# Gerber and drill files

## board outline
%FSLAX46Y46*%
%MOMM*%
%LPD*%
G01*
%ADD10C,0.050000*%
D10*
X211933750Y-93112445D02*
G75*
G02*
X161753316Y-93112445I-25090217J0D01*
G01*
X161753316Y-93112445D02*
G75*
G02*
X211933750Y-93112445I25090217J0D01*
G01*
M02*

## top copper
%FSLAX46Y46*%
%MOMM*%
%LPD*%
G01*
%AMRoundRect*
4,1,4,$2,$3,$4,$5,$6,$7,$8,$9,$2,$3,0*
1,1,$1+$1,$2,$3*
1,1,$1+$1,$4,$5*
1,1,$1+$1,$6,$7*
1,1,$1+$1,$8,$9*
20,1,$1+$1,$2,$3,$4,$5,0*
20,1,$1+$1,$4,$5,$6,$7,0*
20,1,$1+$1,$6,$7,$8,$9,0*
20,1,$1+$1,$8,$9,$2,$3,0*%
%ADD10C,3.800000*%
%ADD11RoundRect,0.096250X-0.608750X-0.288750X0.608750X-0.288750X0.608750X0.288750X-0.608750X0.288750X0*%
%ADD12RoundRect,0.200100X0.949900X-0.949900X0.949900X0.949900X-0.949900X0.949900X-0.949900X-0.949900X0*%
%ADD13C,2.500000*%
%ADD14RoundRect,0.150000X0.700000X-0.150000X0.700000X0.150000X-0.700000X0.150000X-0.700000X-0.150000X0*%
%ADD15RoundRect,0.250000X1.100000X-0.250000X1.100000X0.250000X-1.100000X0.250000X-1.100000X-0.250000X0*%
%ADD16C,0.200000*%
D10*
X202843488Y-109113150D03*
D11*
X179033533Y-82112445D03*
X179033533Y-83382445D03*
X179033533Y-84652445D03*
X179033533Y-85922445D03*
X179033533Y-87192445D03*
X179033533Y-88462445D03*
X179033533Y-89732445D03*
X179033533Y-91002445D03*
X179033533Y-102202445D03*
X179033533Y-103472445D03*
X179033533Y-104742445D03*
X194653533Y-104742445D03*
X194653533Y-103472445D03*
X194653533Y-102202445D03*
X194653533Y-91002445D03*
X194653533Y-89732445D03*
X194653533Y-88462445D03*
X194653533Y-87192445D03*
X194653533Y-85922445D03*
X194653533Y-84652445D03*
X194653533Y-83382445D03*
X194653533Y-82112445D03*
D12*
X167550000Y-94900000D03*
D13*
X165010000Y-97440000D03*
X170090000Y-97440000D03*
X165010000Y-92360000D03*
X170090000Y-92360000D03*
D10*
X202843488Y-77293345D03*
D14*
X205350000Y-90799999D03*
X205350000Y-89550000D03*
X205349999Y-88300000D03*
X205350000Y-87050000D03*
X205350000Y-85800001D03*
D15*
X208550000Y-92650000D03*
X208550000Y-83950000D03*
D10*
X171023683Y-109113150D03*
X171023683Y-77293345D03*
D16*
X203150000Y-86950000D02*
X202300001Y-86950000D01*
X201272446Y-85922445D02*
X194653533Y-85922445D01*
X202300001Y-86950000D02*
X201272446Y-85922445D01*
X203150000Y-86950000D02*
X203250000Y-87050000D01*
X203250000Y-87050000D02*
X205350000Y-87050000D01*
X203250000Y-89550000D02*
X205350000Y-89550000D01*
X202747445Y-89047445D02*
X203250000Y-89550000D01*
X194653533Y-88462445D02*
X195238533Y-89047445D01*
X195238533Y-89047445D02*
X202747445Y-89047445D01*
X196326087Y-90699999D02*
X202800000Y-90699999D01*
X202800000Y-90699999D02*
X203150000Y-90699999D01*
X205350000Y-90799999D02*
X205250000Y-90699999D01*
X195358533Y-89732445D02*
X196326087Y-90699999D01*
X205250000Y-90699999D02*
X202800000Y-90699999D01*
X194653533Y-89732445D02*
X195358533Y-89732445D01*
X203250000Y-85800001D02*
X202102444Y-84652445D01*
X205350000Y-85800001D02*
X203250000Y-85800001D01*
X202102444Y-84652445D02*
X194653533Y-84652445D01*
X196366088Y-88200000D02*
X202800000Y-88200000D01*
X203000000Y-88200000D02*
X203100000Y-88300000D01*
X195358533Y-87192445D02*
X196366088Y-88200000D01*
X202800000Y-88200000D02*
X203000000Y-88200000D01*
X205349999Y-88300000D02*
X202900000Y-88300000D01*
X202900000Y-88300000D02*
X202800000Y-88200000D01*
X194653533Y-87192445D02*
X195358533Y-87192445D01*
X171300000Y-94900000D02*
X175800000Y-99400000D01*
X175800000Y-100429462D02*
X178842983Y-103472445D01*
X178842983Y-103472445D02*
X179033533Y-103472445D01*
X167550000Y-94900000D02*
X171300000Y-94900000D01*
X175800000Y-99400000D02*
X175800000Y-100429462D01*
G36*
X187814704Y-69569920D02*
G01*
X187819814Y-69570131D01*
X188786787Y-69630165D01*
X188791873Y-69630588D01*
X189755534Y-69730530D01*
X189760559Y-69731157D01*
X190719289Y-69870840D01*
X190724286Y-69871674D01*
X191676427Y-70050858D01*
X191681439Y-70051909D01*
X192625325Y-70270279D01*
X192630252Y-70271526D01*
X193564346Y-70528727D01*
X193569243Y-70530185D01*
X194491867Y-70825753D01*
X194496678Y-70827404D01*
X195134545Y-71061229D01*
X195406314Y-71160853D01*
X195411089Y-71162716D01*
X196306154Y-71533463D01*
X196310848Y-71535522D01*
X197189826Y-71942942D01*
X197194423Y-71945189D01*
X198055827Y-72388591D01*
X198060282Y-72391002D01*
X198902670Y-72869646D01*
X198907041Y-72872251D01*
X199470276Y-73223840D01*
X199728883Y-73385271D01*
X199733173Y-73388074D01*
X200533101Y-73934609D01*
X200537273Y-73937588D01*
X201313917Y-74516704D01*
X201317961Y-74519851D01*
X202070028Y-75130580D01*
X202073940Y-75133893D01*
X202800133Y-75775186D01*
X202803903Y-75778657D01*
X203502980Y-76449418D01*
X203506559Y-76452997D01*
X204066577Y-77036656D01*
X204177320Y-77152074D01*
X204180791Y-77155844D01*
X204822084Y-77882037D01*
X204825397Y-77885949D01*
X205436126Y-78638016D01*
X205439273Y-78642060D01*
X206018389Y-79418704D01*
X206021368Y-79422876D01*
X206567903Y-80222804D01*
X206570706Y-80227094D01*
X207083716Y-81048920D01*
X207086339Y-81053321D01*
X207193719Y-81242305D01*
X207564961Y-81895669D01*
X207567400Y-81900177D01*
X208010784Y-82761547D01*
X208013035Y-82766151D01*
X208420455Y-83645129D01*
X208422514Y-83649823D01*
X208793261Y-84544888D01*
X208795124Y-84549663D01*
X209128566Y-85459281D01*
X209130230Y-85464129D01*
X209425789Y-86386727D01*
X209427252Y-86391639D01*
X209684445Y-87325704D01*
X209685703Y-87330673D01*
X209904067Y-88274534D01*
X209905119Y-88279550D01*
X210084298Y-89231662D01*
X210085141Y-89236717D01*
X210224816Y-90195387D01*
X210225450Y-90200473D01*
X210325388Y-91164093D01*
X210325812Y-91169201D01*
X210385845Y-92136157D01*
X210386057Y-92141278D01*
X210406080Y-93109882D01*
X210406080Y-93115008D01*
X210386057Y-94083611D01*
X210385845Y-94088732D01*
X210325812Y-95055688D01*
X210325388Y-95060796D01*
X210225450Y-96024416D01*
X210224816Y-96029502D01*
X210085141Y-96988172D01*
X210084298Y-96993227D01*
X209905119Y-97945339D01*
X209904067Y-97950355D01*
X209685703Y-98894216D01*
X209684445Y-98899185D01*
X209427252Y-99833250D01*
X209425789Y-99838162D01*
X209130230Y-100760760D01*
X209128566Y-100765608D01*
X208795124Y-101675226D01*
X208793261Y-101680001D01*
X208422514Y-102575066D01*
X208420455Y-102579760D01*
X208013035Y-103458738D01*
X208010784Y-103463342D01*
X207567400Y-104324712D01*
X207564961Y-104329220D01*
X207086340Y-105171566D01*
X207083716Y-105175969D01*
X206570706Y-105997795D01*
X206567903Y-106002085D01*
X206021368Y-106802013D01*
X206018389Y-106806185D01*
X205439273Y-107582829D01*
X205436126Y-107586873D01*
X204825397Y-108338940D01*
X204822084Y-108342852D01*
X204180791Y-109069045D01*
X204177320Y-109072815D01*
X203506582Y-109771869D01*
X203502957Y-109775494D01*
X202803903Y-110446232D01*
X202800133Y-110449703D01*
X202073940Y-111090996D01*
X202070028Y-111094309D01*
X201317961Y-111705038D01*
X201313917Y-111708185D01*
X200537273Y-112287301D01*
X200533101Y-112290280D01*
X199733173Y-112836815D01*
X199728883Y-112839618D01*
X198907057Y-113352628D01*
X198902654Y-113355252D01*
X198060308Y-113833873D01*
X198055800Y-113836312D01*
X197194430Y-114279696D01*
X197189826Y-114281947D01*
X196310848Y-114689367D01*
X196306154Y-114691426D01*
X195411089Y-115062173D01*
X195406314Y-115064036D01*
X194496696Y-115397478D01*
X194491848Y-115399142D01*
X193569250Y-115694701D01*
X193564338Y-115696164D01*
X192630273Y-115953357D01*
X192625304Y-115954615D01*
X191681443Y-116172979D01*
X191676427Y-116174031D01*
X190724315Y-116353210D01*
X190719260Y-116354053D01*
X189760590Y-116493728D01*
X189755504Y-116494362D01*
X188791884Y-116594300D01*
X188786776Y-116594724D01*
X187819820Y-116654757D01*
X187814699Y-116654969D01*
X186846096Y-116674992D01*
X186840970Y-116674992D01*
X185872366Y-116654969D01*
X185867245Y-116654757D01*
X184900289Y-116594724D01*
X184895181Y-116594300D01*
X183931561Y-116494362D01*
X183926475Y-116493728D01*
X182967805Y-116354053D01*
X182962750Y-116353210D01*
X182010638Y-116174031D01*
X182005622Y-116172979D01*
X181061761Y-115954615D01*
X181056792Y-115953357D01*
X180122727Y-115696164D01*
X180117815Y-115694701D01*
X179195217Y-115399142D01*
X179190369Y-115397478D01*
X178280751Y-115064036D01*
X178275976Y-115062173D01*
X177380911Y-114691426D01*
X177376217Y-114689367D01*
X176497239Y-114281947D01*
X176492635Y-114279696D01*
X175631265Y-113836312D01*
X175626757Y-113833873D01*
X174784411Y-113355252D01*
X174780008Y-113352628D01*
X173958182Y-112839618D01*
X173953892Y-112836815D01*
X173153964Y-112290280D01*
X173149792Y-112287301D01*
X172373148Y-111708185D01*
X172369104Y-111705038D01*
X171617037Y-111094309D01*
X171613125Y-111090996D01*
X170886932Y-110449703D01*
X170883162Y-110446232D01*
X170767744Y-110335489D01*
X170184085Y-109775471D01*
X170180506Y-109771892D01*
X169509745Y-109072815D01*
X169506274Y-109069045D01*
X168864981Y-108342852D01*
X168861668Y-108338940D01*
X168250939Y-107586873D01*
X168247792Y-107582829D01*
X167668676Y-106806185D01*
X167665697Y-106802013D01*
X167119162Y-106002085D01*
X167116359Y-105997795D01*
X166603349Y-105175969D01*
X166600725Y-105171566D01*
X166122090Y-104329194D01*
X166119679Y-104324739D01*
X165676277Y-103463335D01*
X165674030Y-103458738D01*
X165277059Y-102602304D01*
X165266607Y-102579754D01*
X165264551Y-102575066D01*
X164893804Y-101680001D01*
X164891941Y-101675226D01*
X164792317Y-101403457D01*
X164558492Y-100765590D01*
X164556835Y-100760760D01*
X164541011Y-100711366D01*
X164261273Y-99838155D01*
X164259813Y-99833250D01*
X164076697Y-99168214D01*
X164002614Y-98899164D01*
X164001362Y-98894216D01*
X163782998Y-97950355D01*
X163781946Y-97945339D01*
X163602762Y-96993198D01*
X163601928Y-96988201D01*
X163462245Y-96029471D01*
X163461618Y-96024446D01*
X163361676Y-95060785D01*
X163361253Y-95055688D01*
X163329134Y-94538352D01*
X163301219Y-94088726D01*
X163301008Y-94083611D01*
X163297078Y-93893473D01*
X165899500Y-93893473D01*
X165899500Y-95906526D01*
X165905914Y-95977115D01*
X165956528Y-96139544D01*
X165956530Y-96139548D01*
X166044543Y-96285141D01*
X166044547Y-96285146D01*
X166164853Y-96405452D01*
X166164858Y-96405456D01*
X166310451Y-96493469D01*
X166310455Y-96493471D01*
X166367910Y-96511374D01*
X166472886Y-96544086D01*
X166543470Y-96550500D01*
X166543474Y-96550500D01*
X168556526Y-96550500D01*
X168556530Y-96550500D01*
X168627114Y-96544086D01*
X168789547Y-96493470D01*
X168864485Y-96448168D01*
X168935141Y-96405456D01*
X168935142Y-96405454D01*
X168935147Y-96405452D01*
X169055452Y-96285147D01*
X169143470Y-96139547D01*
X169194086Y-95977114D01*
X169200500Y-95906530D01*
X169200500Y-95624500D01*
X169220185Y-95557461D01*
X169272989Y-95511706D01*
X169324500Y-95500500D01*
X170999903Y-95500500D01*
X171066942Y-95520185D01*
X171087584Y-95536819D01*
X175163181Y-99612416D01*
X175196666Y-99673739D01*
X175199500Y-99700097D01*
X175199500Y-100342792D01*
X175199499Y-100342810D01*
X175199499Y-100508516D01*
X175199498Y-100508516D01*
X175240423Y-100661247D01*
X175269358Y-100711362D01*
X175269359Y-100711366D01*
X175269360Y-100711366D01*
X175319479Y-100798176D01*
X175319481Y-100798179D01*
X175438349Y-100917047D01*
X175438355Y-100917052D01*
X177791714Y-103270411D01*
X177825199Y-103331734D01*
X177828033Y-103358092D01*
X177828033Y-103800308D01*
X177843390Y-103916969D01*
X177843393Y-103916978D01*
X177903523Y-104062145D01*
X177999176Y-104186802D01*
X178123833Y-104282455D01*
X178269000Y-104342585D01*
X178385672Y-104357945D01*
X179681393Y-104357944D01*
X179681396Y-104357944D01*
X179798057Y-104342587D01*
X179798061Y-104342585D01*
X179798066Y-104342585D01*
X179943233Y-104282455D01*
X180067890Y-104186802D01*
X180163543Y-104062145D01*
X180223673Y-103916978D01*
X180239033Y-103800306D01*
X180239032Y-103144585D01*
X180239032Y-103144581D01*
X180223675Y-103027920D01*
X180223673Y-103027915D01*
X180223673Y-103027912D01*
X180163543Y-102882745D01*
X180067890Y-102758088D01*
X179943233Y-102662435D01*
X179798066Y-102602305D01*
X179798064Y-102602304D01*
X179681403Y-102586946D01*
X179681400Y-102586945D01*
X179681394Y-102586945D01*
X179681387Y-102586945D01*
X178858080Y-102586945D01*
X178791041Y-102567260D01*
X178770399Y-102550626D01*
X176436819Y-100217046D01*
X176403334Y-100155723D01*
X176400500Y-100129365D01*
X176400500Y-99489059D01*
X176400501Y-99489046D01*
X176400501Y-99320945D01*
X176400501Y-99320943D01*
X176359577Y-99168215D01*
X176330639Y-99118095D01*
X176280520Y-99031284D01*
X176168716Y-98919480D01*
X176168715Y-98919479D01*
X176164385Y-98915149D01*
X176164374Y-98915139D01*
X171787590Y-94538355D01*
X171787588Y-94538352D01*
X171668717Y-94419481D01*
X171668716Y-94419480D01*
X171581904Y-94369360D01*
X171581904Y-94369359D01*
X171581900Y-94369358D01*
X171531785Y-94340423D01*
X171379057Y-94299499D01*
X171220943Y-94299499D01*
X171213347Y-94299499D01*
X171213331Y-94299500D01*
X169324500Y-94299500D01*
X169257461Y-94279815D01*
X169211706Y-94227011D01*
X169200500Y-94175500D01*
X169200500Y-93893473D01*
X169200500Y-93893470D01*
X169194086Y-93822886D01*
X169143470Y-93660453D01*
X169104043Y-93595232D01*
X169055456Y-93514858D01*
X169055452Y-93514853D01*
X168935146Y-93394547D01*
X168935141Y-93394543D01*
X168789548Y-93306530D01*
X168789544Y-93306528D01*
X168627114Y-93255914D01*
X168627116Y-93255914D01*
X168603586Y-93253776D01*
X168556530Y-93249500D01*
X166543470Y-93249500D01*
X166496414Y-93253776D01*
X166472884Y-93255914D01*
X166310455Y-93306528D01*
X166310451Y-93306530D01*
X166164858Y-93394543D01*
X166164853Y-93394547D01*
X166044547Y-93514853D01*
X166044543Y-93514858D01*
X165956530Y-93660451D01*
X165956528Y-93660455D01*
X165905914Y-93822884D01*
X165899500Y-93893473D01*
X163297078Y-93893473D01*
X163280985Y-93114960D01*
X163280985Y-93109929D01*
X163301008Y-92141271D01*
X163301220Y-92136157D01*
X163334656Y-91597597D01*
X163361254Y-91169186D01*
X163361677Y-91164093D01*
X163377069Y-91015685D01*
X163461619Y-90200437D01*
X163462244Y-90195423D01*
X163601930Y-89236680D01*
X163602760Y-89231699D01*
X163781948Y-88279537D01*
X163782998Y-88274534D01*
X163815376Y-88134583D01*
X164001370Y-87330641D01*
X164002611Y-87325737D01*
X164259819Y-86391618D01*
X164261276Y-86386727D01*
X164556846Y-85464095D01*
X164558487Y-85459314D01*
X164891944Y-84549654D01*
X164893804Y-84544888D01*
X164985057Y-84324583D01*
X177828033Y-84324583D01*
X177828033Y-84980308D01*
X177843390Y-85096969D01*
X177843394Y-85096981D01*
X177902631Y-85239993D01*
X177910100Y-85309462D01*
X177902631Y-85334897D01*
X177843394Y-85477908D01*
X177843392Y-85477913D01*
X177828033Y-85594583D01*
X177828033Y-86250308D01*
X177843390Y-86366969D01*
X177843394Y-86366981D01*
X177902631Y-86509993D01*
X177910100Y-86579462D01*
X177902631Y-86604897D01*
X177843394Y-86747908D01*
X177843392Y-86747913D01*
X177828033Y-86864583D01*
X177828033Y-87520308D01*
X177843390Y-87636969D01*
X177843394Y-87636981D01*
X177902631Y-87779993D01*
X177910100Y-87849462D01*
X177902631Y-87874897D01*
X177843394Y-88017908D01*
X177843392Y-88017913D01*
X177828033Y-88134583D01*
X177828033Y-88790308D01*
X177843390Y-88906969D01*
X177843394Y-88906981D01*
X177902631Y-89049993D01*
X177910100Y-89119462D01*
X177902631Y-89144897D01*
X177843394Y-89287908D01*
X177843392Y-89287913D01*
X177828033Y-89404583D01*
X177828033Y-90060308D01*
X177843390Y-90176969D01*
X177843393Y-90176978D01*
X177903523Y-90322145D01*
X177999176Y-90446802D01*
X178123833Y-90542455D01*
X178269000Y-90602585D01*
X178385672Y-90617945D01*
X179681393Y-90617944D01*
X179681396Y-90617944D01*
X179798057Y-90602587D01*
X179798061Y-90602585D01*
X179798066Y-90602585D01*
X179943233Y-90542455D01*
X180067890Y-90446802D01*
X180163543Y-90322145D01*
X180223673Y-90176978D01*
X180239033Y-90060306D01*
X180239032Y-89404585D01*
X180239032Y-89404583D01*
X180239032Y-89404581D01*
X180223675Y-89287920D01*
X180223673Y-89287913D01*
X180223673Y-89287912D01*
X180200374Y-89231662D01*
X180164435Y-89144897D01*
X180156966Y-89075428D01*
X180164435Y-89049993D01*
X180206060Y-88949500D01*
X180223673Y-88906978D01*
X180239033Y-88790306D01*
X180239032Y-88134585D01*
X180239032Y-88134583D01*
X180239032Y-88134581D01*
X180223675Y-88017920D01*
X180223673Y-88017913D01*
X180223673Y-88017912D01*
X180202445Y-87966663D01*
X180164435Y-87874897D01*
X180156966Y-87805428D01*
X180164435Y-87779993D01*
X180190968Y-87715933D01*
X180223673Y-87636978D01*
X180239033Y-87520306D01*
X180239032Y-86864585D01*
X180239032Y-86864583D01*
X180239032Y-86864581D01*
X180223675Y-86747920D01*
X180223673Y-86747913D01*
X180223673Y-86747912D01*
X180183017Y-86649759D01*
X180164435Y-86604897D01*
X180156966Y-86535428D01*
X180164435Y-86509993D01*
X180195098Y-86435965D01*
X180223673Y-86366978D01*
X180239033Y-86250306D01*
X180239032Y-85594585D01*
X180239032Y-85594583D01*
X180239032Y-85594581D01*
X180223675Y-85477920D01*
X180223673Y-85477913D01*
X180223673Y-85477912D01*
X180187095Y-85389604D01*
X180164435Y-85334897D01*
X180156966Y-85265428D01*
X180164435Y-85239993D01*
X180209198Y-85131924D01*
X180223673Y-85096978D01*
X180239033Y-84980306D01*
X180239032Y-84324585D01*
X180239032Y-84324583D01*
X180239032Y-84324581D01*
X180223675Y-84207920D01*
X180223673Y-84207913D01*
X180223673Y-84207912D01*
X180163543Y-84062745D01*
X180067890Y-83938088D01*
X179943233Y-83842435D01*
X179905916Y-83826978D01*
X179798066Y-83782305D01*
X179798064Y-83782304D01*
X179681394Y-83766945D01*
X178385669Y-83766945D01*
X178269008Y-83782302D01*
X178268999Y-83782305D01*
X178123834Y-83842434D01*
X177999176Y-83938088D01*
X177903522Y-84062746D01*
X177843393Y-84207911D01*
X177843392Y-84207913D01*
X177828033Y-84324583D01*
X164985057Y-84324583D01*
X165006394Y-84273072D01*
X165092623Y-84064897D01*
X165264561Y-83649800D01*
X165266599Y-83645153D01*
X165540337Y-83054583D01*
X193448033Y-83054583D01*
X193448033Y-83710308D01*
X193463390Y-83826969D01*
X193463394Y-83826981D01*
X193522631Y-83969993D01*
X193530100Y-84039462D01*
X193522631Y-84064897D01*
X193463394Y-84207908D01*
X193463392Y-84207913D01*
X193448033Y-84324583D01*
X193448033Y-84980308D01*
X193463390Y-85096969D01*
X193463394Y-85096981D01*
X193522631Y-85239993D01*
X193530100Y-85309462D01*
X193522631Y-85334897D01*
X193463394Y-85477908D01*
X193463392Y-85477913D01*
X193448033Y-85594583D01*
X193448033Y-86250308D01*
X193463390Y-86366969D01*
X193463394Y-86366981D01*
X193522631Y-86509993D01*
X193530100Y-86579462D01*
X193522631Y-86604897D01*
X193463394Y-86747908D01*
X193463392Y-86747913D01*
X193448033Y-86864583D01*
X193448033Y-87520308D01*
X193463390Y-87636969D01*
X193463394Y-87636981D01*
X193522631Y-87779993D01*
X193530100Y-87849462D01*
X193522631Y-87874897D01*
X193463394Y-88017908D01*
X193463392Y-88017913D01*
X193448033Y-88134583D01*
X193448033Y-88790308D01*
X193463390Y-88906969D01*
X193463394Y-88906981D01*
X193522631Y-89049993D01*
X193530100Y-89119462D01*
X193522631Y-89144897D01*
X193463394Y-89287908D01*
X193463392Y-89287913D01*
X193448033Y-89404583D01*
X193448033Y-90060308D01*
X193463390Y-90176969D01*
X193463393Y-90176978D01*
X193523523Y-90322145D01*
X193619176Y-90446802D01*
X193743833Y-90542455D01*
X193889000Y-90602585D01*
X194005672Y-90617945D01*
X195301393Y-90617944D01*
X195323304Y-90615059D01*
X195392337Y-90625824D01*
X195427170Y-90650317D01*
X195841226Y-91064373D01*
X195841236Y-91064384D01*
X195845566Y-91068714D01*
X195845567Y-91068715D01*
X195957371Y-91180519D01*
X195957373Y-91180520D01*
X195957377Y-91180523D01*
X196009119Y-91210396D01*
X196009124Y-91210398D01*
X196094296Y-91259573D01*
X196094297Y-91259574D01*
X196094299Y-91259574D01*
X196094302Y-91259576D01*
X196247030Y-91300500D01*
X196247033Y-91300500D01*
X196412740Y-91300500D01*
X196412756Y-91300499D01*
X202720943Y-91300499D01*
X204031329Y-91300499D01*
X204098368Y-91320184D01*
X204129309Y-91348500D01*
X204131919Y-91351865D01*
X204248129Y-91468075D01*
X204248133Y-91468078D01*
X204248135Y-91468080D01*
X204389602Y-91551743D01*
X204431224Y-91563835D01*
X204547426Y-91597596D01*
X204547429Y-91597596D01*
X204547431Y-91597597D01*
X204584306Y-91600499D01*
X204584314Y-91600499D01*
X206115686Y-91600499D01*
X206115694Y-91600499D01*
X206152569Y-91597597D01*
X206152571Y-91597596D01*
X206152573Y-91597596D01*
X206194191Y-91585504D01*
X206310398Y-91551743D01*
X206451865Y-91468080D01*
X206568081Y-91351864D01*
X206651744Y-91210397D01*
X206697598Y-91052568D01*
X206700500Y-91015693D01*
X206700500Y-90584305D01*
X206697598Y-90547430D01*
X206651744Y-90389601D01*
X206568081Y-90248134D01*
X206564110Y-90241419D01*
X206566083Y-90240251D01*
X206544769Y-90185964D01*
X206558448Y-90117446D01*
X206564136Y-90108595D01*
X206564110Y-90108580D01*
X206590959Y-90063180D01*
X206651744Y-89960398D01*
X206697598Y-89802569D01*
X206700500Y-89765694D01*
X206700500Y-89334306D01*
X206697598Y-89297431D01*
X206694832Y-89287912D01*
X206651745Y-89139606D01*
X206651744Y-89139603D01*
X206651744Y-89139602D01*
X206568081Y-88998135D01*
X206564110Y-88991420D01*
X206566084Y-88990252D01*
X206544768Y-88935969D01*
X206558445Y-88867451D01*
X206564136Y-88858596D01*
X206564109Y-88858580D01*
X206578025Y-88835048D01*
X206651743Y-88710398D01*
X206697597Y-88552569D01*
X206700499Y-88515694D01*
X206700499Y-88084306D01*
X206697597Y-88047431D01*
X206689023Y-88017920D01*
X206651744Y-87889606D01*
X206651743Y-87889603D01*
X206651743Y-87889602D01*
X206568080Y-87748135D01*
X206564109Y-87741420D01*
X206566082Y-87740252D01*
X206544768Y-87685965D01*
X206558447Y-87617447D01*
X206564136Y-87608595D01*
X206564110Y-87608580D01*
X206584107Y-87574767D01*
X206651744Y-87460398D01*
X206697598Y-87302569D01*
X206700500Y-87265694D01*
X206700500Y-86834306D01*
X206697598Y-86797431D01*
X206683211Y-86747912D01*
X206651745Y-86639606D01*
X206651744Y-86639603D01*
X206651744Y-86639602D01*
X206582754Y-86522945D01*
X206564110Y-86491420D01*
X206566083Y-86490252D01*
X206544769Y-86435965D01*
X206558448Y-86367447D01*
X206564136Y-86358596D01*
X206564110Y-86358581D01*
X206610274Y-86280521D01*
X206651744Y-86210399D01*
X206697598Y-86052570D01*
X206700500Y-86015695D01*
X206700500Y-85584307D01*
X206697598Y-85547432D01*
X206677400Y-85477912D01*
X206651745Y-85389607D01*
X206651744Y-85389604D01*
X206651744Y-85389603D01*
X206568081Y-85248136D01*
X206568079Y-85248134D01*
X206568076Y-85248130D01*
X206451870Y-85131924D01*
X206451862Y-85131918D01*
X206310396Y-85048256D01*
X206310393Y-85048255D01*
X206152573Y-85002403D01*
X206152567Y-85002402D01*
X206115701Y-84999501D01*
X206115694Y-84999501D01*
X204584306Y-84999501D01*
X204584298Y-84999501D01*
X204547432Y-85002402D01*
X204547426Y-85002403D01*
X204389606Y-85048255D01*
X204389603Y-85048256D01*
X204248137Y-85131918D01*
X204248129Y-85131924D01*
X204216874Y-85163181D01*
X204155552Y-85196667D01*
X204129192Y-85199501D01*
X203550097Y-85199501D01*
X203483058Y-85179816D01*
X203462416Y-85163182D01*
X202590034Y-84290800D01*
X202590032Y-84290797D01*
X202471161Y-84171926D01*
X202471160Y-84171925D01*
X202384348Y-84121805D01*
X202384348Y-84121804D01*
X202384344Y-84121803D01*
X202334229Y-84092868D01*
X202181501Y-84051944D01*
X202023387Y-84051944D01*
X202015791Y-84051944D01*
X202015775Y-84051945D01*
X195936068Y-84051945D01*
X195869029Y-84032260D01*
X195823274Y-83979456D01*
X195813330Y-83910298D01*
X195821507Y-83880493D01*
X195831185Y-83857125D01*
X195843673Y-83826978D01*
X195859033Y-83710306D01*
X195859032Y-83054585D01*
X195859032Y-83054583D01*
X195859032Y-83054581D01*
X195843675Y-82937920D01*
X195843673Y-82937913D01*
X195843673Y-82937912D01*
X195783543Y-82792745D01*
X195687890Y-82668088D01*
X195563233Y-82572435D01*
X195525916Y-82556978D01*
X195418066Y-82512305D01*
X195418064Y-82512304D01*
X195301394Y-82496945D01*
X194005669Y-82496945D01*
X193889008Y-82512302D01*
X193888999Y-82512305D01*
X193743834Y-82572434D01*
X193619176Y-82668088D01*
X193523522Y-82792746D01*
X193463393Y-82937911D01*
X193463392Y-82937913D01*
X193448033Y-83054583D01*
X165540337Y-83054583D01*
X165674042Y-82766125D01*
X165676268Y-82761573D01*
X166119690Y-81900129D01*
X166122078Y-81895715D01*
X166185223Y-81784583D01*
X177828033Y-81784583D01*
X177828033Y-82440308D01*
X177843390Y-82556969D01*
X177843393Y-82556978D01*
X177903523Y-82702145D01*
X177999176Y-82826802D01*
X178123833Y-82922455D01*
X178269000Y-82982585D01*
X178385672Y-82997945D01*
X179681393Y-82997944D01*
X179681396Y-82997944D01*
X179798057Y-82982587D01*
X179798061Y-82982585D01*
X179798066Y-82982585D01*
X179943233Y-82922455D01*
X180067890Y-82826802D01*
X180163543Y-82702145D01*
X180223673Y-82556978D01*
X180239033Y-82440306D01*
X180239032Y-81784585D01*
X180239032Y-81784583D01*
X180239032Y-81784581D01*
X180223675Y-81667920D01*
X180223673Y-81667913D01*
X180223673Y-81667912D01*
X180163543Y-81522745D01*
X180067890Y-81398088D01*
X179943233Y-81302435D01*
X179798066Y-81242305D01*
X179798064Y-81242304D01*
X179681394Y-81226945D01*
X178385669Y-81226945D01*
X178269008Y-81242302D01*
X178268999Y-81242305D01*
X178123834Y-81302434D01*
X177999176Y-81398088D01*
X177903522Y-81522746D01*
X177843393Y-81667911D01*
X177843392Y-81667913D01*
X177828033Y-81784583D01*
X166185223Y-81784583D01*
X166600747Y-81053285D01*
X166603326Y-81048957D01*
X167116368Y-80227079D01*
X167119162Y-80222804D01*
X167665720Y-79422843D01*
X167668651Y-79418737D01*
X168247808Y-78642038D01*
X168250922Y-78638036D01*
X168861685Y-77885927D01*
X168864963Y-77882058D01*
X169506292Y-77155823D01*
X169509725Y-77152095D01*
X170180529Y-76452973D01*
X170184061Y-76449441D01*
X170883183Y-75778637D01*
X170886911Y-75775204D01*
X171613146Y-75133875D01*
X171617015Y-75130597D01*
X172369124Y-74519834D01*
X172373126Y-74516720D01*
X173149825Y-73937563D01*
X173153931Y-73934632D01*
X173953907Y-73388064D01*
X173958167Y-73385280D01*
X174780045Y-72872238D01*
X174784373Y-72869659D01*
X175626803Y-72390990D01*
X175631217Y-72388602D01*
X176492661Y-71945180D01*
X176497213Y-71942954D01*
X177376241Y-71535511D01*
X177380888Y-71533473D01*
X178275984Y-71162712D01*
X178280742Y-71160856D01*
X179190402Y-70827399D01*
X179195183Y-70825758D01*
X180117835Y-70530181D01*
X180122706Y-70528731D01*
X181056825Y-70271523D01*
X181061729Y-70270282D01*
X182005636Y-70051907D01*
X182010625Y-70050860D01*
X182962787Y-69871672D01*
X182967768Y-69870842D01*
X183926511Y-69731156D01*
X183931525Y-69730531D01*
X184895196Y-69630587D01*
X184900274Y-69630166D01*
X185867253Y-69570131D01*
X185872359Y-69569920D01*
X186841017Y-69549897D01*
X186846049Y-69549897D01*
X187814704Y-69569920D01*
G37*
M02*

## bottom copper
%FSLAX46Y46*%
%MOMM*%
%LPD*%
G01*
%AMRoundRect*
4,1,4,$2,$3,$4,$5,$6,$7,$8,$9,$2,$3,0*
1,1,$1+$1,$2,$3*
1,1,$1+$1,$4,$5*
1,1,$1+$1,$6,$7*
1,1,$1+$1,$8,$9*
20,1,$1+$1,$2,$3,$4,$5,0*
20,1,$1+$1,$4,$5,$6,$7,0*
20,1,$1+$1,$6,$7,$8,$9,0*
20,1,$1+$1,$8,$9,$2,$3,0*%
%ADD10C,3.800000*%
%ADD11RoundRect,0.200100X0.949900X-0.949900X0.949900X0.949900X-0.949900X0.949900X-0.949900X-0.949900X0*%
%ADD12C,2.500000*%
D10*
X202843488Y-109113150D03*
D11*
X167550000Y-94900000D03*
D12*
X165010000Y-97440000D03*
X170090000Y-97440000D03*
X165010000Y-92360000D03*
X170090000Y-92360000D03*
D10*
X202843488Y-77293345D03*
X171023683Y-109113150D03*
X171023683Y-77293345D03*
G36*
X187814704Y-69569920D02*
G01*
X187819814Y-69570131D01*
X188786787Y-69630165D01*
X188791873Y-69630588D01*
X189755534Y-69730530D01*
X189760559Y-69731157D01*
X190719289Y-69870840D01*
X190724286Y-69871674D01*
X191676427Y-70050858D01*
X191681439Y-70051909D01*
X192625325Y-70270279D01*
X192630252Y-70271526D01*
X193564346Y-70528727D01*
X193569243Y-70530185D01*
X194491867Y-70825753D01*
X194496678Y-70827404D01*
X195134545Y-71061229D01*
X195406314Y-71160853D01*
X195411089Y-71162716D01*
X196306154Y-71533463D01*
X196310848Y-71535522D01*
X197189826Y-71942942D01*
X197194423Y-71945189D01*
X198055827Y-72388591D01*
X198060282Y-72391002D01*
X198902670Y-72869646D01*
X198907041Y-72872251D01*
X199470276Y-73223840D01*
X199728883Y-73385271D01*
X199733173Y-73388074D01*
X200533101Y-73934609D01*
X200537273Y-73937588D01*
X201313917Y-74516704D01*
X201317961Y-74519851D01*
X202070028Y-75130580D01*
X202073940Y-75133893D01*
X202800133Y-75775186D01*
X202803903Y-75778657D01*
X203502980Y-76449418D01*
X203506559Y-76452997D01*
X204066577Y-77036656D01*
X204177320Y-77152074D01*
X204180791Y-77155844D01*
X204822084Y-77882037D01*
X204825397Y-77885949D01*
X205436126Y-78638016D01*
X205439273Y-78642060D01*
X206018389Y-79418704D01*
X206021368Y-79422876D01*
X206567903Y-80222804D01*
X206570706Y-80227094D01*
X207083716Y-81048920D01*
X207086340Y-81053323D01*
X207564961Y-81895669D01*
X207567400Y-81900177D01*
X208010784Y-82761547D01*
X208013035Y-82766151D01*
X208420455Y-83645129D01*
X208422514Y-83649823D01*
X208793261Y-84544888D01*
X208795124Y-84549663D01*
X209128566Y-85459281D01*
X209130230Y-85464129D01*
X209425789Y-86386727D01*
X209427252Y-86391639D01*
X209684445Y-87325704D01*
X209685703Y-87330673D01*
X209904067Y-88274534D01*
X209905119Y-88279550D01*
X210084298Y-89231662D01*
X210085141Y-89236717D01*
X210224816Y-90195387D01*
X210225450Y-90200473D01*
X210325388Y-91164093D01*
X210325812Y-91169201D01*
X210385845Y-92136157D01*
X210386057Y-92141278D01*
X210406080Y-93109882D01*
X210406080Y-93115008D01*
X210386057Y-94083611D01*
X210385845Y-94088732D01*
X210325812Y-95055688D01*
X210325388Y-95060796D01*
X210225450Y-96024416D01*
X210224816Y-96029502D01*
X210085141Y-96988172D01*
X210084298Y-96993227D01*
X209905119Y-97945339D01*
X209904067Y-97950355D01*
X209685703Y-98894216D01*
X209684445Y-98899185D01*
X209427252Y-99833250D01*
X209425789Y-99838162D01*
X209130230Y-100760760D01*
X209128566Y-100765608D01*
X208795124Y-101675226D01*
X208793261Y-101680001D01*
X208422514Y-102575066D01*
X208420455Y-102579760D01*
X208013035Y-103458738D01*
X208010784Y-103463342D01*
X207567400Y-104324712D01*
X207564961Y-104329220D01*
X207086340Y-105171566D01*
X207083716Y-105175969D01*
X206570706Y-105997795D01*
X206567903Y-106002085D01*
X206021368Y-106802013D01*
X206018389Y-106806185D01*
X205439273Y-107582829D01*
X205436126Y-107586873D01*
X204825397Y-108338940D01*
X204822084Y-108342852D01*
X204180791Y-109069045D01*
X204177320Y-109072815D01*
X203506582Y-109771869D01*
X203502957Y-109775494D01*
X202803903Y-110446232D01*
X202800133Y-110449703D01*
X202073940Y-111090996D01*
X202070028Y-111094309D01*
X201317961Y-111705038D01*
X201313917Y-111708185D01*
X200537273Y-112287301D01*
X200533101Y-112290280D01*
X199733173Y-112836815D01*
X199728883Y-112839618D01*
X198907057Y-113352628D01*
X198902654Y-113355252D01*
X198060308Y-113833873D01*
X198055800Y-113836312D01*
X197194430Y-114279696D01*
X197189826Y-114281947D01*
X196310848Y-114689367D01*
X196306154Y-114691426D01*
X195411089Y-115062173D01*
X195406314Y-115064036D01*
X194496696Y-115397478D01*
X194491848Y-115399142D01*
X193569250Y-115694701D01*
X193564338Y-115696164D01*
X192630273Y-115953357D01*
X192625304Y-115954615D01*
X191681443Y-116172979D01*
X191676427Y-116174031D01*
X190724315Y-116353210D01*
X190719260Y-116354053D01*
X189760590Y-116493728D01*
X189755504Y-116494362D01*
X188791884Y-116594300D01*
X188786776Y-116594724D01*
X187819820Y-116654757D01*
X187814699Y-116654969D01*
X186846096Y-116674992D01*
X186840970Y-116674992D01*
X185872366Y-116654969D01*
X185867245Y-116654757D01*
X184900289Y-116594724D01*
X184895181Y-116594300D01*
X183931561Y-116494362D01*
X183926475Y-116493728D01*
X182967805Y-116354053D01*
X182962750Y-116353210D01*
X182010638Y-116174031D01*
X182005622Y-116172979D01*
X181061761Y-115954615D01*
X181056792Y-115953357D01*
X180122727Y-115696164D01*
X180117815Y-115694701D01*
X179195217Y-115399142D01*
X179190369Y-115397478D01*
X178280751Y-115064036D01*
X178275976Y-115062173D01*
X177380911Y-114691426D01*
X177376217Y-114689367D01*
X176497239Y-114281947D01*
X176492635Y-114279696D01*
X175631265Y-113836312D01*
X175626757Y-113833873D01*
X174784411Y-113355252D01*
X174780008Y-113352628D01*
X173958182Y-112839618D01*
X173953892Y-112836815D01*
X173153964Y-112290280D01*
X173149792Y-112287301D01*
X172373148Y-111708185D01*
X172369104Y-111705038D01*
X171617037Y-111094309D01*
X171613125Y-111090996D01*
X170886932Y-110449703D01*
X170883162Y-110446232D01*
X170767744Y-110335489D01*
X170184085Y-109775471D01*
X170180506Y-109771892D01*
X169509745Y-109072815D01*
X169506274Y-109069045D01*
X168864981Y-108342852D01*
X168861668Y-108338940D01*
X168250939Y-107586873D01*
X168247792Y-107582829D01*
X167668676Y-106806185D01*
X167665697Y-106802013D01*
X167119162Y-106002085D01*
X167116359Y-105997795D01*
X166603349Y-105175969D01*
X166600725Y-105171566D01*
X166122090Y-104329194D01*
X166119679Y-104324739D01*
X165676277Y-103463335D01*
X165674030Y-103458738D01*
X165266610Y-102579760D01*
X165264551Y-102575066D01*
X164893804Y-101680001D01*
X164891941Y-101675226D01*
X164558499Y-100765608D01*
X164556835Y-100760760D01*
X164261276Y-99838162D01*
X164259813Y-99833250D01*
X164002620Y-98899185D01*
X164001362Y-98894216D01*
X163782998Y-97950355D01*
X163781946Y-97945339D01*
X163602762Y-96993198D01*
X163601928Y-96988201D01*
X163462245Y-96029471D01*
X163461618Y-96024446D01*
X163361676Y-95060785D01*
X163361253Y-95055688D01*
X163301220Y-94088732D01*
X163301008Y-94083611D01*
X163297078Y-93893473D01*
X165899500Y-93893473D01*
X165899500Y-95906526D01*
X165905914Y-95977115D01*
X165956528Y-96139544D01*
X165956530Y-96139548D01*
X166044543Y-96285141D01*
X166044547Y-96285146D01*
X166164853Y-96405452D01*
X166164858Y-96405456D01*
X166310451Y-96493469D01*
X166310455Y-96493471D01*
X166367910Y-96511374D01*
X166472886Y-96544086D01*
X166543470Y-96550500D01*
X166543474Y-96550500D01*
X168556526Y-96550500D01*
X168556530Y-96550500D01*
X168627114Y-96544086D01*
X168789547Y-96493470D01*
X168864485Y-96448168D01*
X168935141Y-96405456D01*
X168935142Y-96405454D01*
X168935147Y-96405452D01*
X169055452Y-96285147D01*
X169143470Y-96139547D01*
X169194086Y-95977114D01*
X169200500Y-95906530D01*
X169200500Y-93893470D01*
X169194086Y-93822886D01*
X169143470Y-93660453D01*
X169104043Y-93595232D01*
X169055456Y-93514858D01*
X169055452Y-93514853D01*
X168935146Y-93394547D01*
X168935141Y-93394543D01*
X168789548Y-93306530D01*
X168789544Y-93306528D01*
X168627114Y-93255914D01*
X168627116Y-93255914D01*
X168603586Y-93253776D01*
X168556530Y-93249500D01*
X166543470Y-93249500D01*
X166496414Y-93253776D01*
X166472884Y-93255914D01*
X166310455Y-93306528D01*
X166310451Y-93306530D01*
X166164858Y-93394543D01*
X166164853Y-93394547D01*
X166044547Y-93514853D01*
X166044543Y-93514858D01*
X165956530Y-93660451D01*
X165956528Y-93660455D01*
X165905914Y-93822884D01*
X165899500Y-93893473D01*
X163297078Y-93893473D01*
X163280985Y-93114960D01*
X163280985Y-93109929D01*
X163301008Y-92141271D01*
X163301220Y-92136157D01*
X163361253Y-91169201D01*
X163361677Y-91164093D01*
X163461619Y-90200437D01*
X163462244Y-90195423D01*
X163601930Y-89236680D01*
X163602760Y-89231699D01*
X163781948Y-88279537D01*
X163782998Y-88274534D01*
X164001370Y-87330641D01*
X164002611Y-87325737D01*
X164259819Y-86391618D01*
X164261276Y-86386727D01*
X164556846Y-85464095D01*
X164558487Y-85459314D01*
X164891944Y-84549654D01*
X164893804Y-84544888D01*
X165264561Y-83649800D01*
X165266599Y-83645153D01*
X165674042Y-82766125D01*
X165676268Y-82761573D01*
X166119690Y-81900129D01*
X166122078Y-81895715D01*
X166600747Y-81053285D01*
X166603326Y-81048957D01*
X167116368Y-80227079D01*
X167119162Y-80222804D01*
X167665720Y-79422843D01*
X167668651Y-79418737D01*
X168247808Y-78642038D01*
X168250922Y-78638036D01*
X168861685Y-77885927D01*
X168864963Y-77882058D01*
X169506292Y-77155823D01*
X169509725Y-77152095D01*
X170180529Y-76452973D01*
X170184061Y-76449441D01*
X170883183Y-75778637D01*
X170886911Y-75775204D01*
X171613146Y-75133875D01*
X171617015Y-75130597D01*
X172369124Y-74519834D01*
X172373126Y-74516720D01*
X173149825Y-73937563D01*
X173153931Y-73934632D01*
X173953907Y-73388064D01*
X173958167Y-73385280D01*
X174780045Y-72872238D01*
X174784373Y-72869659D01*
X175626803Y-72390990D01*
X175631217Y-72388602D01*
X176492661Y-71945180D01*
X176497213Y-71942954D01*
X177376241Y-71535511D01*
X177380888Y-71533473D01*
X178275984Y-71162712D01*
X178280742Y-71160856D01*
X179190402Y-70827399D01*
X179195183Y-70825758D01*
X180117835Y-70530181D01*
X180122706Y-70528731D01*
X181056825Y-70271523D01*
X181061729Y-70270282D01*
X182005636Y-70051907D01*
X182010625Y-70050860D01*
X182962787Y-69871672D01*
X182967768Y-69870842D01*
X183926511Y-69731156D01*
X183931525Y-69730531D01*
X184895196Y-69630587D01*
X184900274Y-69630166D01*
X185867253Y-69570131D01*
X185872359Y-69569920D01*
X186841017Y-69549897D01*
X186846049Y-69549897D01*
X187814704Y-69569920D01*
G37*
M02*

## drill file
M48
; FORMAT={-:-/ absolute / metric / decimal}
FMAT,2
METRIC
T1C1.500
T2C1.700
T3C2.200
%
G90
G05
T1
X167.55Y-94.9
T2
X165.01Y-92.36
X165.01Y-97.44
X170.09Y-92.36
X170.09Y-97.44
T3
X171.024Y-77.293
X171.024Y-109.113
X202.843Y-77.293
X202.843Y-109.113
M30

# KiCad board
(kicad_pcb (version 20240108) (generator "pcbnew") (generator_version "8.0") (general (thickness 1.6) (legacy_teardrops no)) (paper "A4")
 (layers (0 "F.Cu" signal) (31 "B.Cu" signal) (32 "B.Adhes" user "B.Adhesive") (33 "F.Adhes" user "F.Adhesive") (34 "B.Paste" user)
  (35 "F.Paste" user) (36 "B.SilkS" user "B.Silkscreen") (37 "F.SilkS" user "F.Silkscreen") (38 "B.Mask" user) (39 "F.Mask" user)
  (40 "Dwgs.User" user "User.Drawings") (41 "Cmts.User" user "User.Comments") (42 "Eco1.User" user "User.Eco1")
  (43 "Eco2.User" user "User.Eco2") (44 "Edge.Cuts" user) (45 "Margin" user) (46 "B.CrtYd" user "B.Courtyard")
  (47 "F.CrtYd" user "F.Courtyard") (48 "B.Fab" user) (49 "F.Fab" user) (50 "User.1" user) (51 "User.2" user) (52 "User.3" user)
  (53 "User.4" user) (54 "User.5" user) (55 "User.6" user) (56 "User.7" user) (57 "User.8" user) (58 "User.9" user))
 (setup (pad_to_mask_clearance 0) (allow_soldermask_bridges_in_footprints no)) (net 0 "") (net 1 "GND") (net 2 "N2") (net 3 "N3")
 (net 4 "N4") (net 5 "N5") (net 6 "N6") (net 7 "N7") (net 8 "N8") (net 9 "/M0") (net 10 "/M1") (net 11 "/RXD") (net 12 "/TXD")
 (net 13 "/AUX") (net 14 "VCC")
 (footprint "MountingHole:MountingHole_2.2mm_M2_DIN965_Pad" (layer "F.Cu") (at 202.843488 109.11315)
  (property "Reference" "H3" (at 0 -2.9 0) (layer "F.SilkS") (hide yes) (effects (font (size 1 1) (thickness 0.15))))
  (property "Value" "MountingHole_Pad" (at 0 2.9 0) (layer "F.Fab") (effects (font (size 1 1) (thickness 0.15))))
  (pad "1" thru_hole circle (at 0 0) (size 3.8 3.8) (drill 2.2) (layers "*.Cu" "*.Mask") (remove_unused_layers no) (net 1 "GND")))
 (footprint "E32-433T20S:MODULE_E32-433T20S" (layer "F.Cu") (at 186.843533 93.112445)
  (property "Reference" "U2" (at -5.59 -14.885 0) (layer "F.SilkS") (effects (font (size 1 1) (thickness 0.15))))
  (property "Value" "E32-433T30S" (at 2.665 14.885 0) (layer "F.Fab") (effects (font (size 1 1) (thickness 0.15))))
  (pad "1" smd roundrect (at -7.81 -11) (size 1.41 0.77) (layers "F.Cu" "F.Paste" "F.Mask") (roundrect_rratio 0.125) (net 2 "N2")
   (solder_mask_margin 0.102))
  (pad "2" smd roundrect (at -7.81 -9.73) (size 1.41 0.77) (layers "F.Cu" "F.Paste" "F.Mask") (roundrect_rratio 0.125) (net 1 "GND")
   (solder_mask_margin 0.102))
  (pad "3" smd roundrect (at -7.81 -8.46) (size 1.41 0.77) (layers "F.Cu" "F.Paste" "F.Mask") (roundrect_rratio 0.125) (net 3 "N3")
   (solder_mask_margin 0.102))
  (pad "4" smd roundrect (at -7.81 -7.19) (size 1.41 0.77) (layers "F.Cu" "F.Paste" "F.Mask") (roundrect_rratio 0.125) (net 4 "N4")
   (solder_mask_margin 0.102))
  (pad "5" smd roundrect (at -7.81 -5.92) (size 1.41 0.77) (layers "F.Cu" "F.Paste" "F.Mask") (roundrect_rratio 0.125) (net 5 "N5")
   (solder_mask_margin 0.102))
  (pad "6" smd roundrect (at -7.81 -4.65) (size 1.41 0.77) (layers "F.Cu" "F.Paste" "F.Mask") (roundrect_rratio 0.125) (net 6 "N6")
   (solder_mask_margin 0.102))
  (pad "7" smd roundrect (at -7.81 -3.38) (size 1.41 0.77) (layers "F.Cu" "F.Paste" "F.Mask") (roundrect_rratio 0.125) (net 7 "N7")
   (solder_mask_margin 0.102))
  (pad "8" smd roundrect (at -7.81 -2.11) (size 1.41 0.77) (layers "F.Cu" "F.Paste" "F.Mask") (roundrect_rratio 0.125) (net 1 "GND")
   (solder_mask_margin 0.102))
  (pad "11" smd roundrect (at -7.81 9.09) (size 1.41 0.77) (layers "F.Cu" "F.Paste" "F.Mask") (roundrect_rratio 0.125) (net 1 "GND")
   (solder_mask_margin 0.102))
  (pad "12" smd roundrect (at -7.81 10.36) (size 1.41 0.77) (layers "F.Cu" "F.Paste" "F.Mask") (roundrect_rratio 0.125) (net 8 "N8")
   (solder_mask_margin 0.102))
  (pad "13" smd roundrect (at -7.81 11.63) (size 1.41 0.77) (layers "F.Cu" "F.Paste" "F.Mask") (roundrect_rratio 0.125) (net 1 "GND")
   (solder_mask_margin 0.102))
  (pad "14" smd roundrect (at 7.81 11.63) (size 1.41 0.77) (layers "F.Cu" "F.Paste" "F.Mask") (roundrect_rratio 0.125) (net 1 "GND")
   (solder_mask_margin 0.102))
  (pad "15" smd roundrect (at 7.81 10.36) (size 1.41 0.77) (layers "F.Cu" "F.Paste" "F.Mask") (roundrect_rratio 0.125) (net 1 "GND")
   (solder_mask_margin 0.102))
  (pad "16" smd roundrect (at 7.81 9.09) (size 1.41 0.77) (layers "F.Cu" "F.Paste" "F.Mask") (roundrect_rratio 0.125) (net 1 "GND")
   (solder_mask_margin 0.102))
  (pad "19" smd roundrect (at 7.81 -2.11) (size 1.41 0.77) (layers "F.Cu" "F.Paste" "F.Mask") (roundrect_rratio 0.125) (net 1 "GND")
   (solder_mask_margin 0.102))
  (pad "20" smd roundrect (at 7.81 -3.38) (size 1.41 0.77) (layers "F.Cu" "F.Paste" "F.Mask") (roundrect_rratio 0.125) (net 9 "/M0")
   (solder_mask_margin 0.102))
  (pad "21" smd roundrect (at 7.81 -4.65) (size 1.41 0.77) (layers "F.Cu" "F.Paste" "F.Mask") (roundrect_rratio 0.125) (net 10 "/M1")
   (solder_mask_margin 0.102))
  (pad "22" smd roundrect (at 7.81 -5.92) (size 1.41 0.77) (layers "F.Cu" "F.Paste" "F.Mask") (roundrect_rratio 0.125) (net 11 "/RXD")
   (solder_mask_margin 0.102))
  (pad "23" smd roundrect (at 7.81 -7.19) (size 1.41 0.77) (layers "F.Cu" "F.Paste" "F.Mask") (roundrect_rratio 0.125) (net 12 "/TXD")
   (solder_mask_margin 0.102))
  (pad "24" smd roundrect (at 7.81 -8.46) (size 1.41 0.77) (layers "F.Cu" "F.Paste" "F.Mask") (roundrect_rratio 0.125) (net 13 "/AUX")
   (solder_mask_margin 0.102))
  (pad "25" smd roundrect (at 7.81 -9.73) (size 1.41 0.77) (layers "F.Cu" "F.Paste" "F.Mask") (roundrect_rratio 0.125) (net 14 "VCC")
   (solder_mask_margin 0.102))
  (pad "26" smd roundrect (at 7.81 -11) (size 1.41 0.77) (layers "F.Cu" "F.Paste" "F.Mask") (roundrect_rratio 0.125) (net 1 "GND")
   (solder_mask_margin 0.102)))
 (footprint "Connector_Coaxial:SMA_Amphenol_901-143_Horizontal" (layer "F.Cu") (at 167.55 94.9 90)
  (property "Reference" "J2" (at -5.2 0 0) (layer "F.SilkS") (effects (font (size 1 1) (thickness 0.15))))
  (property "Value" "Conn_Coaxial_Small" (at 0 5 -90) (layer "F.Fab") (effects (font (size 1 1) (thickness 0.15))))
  (pad "1" thru_hole roundrect (at 0 0 90) (size 2.3 2.3) (drill 1.5) (layers "*.Cu" "*.Mask") (remove_unused_layers yes)
   (keep_end_layers yes) (zone_layer_connections) (roundrect_rratio 0.087) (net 8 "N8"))
  (pad "2" thru_hole circle (at -2.54 -2.54 90) (size 2.5 2.5) (drill 1.7) (layers "*.Cu" "*.Mask") (remove_unused_layers yes)
   (keep_end_layers yes) (zone_layer_connections) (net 1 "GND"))
  (pad "2" thru_hole circle (at -2.54 2.54 90) (size 2.5 2.5) (drill 1.7) (layers "*.Cu" "*.Mask") (remove_unused_layers yes)
   (keep_end_layers yes) (zone_layer_connections) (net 1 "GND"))
  (pad "2" thru_hole circle (at 2.54 -2.54 90) (size 2.5 2.5) (drill 1.7) (layers "*.Cu" "*.Mask") (remove_unused_layers yes)
   (keep_end_layers yes) (zone_layer_connections) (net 1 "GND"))
  (pad "2" thru_hole circle (at 2.54 2.54 90) (size 2.5 2.5) (drill 1.7) (layers "*.Cu" "*.Mask") (remove_unused_layers yes)
   (keep_end_layers yes) (zone_layer_connections) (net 1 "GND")))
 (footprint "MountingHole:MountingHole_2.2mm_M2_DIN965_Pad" (layer "F.Cu") (at 202.843488 77.293345)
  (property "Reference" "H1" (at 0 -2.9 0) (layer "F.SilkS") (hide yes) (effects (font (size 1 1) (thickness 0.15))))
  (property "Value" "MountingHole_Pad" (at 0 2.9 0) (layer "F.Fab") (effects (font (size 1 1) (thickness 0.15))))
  (pad "1" thru_hole circle (at 0 0) (size 3.8 3.8) (drill 2.2) (layers "*.Cu" "*.Mask") (remove_unused_layers no) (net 1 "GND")))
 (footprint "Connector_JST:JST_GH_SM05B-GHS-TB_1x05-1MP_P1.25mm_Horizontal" (layer "F.Cu") (at 207.2 88.3 90)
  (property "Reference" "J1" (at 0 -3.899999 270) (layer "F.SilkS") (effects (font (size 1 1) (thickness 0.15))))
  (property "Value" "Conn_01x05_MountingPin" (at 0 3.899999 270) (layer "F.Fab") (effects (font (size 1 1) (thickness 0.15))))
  (pad "1" smd roundrect (at -2.499999 -1.85 90) (size 0.6 1.7) (layers "F.Cu" "F.Paste" "F.Mask") (roundrect_rratio 0.25) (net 9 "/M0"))
  (pad "2" smd roundrect (at -1.25 -1.85 90) (size 0.6 1.7) (layers "F.Cu" "F.Paste" "F.Mask") (roundrect_rratio 0.25) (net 10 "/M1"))
  (pad "3" smd roundrect (at 0 -1.850001 90) (size 0.6 1.7) (layers "F.Cu" "F.Paste" "F.Mask") (roundrect_rratio 0.25) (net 11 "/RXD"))
  (pad "4" smd roundrect (at 1.25 -1.85 90) (size 0.6 1.7) (layers "F.Cu" "F.Paste" "F.Mask") (roundrect_rratio 0.25) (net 12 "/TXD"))
  (pad "5" smd roundrect (at 2.499999 -1.85 90) (size 0.6 1.7) (layers "F.Cu" "F.Paste" "F.Mask") (roundrect_rratio 0.25) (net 13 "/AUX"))
  (pad "MP" smd roundrect (at -4.35 1.35 90) (size 1 2.7) (layers "F.Cu" "F.Paste" "F.Mask") (roundrect_rratio 0.25) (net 1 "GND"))
  (pad "MP" smd roundrect (at 4.35 1.35 90) (size 1 2.7) (layers "F.Cu" "F.Paste" "F.Mask") (roundrect_rratio 0.25) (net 1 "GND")))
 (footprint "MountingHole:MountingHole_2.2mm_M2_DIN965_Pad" (layer "F.Cu") (at 171.023683 109.11315)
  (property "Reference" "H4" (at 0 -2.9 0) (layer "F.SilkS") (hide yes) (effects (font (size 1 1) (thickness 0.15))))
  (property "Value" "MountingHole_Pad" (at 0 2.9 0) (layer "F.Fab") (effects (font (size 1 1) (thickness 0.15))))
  (pad "1" thru_hole circle (at 0 0) (size 3.8 3.8) (drill 2.2) (layers "*.Cu" "*.Mask") (remove_unused_layers no) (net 1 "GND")))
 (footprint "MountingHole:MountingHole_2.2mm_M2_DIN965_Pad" (layer "F.Cu") (at 171.023683 77.293345)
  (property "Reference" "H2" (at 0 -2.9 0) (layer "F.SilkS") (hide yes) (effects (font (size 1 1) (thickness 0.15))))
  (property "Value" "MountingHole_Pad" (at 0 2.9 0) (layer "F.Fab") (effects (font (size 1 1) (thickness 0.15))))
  (pad "1" thru_hole circle (at 0 0) (size 3.8 3.8) (drill 2.2) (layers "*.Cu" "*.Mask") (remove_unused_layers no) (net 1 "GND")))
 (gr_circle (center 186.843533 93.112445) (end 211.933586 93.203248) (stroke (width 0.05) (type default)) (fill none) (layer "Edge.Cuts"))
 (segment (start 203.15 86.95) (end 202.300001 86.95) (width 0.2) (layer "F.Cu") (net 12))
 (segment (start 201.272446 85.922445) (end 194.653533 85.922445) (width 0.2) (layer "F.Cu") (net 12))
 (segment (start 202.300001 86.95) (end 201.272446 85.922445) (width 0.2) (layer "F.Cu") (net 12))
 (segment (start 203.15 86.95) (end 203.25 87.05) (width 0.2) (layer "F.Cu") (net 12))
 (segment (start 203.25 87.05) (end 205.35 87.05) (width 0.2) (layer "F.Cu") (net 12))
 (segment (start 203.25 89.55) (end 205.35 89.55) (width 0.2) (layer "F.Cu") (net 10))
 (segment (start 202.747445 89.047445) (end 203.25 89.55) (width 0.2) (layer "F.Cu") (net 10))
 (segment (start 194.653533 88.462445) (end 195.238533 89.047445) (width 0.2) (layer "F.Cu") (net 10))
 (segment (start 195.238533 89.047445) (end 202.747445 89.047445) (width 0.2) (layer "F.Cu") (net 10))
 (segment (start 196.326087 90.699999) (end 202.8 90.699999) (width 0.2) (layer "F.Cu") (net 9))
 (segment (start 202.8 90.699999) (end 203.15 90.699999) (width 0.2) (layer "F.Cu") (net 9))
 (segment (start 205.35 90.799999) (end 205.25 90.699999) (width 0.2) (layer "F.Cu") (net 9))
 (segment (start 195.358533 89.732445) (end 196.326087 90.699999) (width 0.2) (layer "F.Cu") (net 9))
 (segment (start 205.25 90.699999) (end 202.8 90.699999) (width 0.2) (layer "F.Cu") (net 9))
 (segment (start 194.653533 89.732445) (end 195.358533 89.732445) (width 0.2) (layer "F.Cu") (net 9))
 (segment (start 203.25 85.800001) (end 202.102444 84.652445) (width 0.2) (layer "F.Cu") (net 13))
 (segment (start 205.35 85.800001) (end 203.25 85.800001) (width 0.2) (layer "F.Cu") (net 13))
 (segment (start 202.102444 84.652445) (end 194.653533 84.652445) (width 0.2) (layer "F.Cu") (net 13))
 (segment (start 196.366088 88.2) (end 202.8 88.2) (width 0.2) (layer "F.Cu") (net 11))
 (segment (start 203 88.2) (end 203.1 88.3) (width 0.2) (layer "F.Cu") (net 11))
 (segment (start 195.358533 87.192445) (end 196.366088 88.2) (width 0.2) (layer "F.Cu") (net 11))
 (segment (start 202.8 88.2) (end 203 88.2) (width 0.2) (layer "F.Cu") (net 11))
 (segment (start 205.349999 88.3) (end 202.9 88.3) (width 0.2) (layer "F.Cu") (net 11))
 (segment (start 202.9 88.3) (end 202.8 88.2) (width 0.2) (layer "F.Cu") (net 11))
 (segment (start 194.653533 87.192445) (end 195.358533 87.192445) (width 0.2) (layer "F.Cu") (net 11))
 (segment (start 171.3 94.9) (end 175.8 99.4) (width 0.2) (layer "F.Cu") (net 8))
 (segment (start 175.8 100.429462) (end 178.842983 103.472445) (width 0.2) (layer "F.Cu") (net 8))
 (segment (start 178.842983 103.472445) (end 179.033533 103.472445) (width 0.2) (layer "F.Cu") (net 8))
 (segment (start 167.55 94.9) (end 171.3 94.9) (width 0.2) (layer "F.Cu") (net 8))
 (segment (start 175.8 99.4) (end 175.8 100.429462) (width 0.2) (layer "F.Cu") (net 8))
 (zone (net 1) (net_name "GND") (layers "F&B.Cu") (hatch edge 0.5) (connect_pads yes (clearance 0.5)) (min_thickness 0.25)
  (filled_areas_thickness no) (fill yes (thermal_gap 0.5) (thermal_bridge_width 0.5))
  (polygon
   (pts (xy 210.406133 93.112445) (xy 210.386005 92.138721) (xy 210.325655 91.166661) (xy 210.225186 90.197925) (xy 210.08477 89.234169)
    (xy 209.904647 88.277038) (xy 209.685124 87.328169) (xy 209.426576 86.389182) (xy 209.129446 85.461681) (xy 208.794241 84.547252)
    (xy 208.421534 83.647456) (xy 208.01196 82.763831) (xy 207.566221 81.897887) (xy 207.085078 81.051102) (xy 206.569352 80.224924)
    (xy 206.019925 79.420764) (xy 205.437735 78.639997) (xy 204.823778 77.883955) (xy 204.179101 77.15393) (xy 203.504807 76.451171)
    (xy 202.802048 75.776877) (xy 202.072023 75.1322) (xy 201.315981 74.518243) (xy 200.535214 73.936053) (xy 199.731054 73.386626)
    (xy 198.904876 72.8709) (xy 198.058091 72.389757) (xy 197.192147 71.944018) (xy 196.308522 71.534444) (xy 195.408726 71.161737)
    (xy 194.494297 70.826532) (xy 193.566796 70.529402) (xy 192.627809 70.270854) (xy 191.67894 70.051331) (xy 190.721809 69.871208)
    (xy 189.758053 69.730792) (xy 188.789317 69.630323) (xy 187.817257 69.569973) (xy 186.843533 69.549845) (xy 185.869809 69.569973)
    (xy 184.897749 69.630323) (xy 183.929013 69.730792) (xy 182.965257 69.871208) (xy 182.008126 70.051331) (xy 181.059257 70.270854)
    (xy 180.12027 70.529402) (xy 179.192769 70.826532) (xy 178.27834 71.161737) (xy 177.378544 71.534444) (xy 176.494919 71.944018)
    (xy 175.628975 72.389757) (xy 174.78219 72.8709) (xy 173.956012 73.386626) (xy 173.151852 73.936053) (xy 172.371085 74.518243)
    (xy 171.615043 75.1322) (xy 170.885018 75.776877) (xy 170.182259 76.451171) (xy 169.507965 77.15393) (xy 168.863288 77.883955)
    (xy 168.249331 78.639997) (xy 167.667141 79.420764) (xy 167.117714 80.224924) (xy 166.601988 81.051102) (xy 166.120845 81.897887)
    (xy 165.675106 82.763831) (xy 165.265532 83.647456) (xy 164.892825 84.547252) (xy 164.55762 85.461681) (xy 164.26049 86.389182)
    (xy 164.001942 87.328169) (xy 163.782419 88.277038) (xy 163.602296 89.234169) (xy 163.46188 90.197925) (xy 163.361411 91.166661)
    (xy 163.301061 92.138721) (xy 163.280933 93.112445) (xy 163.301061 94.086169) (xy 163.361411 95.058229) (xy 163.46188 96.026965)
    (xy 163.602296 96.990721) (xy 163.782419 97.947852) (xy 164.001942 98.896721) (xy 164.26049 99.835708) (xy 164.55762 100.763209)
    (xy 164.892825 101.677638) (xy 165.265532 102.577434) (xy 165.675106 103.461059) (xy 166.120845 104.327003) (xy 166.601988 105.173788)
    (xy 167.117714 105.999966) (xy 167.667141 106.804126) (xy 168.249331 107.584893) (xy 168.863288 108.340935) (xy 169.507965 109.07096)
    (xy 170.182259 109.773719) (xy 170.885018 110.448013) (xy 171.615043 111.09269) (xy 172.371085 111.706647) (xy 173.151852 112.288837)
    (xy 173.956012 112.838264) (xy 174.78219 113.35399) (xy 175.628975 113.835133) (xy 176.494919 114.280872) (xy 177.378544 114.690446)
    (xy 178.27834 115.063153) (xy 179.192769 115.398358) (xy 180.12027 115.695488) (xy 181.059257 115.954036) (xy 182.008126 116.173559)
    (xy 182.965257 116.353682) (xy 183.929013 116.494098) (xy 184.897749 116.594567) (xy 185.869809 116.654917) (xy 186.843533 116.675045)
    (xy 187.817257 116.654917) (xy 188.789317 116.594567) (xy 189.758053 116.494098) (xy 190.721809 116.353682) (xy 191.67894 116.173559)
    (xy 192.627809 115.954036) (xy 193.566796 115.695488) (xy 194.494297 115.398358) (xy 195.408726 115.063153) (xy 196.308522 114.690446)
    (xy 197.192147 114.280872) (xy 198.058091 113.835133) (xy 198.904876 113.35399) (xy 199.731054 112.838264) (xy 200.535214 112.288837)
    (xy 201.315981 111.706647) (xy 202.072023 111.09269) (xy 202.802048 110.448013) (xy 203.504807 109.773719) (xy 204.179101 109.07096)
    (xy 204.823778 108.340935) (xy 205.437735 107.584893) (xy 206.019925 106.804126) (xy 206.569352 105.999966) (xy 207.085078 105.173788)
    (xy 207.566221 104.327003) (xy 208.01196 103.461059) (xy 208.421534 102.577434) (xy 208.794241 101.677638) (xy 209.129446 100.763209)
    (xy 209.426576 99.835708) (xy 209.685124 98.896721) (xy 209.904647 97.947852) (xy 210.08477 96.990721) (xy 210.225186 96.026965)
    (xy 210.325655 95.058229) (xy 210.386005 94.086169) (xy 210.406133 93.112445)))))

